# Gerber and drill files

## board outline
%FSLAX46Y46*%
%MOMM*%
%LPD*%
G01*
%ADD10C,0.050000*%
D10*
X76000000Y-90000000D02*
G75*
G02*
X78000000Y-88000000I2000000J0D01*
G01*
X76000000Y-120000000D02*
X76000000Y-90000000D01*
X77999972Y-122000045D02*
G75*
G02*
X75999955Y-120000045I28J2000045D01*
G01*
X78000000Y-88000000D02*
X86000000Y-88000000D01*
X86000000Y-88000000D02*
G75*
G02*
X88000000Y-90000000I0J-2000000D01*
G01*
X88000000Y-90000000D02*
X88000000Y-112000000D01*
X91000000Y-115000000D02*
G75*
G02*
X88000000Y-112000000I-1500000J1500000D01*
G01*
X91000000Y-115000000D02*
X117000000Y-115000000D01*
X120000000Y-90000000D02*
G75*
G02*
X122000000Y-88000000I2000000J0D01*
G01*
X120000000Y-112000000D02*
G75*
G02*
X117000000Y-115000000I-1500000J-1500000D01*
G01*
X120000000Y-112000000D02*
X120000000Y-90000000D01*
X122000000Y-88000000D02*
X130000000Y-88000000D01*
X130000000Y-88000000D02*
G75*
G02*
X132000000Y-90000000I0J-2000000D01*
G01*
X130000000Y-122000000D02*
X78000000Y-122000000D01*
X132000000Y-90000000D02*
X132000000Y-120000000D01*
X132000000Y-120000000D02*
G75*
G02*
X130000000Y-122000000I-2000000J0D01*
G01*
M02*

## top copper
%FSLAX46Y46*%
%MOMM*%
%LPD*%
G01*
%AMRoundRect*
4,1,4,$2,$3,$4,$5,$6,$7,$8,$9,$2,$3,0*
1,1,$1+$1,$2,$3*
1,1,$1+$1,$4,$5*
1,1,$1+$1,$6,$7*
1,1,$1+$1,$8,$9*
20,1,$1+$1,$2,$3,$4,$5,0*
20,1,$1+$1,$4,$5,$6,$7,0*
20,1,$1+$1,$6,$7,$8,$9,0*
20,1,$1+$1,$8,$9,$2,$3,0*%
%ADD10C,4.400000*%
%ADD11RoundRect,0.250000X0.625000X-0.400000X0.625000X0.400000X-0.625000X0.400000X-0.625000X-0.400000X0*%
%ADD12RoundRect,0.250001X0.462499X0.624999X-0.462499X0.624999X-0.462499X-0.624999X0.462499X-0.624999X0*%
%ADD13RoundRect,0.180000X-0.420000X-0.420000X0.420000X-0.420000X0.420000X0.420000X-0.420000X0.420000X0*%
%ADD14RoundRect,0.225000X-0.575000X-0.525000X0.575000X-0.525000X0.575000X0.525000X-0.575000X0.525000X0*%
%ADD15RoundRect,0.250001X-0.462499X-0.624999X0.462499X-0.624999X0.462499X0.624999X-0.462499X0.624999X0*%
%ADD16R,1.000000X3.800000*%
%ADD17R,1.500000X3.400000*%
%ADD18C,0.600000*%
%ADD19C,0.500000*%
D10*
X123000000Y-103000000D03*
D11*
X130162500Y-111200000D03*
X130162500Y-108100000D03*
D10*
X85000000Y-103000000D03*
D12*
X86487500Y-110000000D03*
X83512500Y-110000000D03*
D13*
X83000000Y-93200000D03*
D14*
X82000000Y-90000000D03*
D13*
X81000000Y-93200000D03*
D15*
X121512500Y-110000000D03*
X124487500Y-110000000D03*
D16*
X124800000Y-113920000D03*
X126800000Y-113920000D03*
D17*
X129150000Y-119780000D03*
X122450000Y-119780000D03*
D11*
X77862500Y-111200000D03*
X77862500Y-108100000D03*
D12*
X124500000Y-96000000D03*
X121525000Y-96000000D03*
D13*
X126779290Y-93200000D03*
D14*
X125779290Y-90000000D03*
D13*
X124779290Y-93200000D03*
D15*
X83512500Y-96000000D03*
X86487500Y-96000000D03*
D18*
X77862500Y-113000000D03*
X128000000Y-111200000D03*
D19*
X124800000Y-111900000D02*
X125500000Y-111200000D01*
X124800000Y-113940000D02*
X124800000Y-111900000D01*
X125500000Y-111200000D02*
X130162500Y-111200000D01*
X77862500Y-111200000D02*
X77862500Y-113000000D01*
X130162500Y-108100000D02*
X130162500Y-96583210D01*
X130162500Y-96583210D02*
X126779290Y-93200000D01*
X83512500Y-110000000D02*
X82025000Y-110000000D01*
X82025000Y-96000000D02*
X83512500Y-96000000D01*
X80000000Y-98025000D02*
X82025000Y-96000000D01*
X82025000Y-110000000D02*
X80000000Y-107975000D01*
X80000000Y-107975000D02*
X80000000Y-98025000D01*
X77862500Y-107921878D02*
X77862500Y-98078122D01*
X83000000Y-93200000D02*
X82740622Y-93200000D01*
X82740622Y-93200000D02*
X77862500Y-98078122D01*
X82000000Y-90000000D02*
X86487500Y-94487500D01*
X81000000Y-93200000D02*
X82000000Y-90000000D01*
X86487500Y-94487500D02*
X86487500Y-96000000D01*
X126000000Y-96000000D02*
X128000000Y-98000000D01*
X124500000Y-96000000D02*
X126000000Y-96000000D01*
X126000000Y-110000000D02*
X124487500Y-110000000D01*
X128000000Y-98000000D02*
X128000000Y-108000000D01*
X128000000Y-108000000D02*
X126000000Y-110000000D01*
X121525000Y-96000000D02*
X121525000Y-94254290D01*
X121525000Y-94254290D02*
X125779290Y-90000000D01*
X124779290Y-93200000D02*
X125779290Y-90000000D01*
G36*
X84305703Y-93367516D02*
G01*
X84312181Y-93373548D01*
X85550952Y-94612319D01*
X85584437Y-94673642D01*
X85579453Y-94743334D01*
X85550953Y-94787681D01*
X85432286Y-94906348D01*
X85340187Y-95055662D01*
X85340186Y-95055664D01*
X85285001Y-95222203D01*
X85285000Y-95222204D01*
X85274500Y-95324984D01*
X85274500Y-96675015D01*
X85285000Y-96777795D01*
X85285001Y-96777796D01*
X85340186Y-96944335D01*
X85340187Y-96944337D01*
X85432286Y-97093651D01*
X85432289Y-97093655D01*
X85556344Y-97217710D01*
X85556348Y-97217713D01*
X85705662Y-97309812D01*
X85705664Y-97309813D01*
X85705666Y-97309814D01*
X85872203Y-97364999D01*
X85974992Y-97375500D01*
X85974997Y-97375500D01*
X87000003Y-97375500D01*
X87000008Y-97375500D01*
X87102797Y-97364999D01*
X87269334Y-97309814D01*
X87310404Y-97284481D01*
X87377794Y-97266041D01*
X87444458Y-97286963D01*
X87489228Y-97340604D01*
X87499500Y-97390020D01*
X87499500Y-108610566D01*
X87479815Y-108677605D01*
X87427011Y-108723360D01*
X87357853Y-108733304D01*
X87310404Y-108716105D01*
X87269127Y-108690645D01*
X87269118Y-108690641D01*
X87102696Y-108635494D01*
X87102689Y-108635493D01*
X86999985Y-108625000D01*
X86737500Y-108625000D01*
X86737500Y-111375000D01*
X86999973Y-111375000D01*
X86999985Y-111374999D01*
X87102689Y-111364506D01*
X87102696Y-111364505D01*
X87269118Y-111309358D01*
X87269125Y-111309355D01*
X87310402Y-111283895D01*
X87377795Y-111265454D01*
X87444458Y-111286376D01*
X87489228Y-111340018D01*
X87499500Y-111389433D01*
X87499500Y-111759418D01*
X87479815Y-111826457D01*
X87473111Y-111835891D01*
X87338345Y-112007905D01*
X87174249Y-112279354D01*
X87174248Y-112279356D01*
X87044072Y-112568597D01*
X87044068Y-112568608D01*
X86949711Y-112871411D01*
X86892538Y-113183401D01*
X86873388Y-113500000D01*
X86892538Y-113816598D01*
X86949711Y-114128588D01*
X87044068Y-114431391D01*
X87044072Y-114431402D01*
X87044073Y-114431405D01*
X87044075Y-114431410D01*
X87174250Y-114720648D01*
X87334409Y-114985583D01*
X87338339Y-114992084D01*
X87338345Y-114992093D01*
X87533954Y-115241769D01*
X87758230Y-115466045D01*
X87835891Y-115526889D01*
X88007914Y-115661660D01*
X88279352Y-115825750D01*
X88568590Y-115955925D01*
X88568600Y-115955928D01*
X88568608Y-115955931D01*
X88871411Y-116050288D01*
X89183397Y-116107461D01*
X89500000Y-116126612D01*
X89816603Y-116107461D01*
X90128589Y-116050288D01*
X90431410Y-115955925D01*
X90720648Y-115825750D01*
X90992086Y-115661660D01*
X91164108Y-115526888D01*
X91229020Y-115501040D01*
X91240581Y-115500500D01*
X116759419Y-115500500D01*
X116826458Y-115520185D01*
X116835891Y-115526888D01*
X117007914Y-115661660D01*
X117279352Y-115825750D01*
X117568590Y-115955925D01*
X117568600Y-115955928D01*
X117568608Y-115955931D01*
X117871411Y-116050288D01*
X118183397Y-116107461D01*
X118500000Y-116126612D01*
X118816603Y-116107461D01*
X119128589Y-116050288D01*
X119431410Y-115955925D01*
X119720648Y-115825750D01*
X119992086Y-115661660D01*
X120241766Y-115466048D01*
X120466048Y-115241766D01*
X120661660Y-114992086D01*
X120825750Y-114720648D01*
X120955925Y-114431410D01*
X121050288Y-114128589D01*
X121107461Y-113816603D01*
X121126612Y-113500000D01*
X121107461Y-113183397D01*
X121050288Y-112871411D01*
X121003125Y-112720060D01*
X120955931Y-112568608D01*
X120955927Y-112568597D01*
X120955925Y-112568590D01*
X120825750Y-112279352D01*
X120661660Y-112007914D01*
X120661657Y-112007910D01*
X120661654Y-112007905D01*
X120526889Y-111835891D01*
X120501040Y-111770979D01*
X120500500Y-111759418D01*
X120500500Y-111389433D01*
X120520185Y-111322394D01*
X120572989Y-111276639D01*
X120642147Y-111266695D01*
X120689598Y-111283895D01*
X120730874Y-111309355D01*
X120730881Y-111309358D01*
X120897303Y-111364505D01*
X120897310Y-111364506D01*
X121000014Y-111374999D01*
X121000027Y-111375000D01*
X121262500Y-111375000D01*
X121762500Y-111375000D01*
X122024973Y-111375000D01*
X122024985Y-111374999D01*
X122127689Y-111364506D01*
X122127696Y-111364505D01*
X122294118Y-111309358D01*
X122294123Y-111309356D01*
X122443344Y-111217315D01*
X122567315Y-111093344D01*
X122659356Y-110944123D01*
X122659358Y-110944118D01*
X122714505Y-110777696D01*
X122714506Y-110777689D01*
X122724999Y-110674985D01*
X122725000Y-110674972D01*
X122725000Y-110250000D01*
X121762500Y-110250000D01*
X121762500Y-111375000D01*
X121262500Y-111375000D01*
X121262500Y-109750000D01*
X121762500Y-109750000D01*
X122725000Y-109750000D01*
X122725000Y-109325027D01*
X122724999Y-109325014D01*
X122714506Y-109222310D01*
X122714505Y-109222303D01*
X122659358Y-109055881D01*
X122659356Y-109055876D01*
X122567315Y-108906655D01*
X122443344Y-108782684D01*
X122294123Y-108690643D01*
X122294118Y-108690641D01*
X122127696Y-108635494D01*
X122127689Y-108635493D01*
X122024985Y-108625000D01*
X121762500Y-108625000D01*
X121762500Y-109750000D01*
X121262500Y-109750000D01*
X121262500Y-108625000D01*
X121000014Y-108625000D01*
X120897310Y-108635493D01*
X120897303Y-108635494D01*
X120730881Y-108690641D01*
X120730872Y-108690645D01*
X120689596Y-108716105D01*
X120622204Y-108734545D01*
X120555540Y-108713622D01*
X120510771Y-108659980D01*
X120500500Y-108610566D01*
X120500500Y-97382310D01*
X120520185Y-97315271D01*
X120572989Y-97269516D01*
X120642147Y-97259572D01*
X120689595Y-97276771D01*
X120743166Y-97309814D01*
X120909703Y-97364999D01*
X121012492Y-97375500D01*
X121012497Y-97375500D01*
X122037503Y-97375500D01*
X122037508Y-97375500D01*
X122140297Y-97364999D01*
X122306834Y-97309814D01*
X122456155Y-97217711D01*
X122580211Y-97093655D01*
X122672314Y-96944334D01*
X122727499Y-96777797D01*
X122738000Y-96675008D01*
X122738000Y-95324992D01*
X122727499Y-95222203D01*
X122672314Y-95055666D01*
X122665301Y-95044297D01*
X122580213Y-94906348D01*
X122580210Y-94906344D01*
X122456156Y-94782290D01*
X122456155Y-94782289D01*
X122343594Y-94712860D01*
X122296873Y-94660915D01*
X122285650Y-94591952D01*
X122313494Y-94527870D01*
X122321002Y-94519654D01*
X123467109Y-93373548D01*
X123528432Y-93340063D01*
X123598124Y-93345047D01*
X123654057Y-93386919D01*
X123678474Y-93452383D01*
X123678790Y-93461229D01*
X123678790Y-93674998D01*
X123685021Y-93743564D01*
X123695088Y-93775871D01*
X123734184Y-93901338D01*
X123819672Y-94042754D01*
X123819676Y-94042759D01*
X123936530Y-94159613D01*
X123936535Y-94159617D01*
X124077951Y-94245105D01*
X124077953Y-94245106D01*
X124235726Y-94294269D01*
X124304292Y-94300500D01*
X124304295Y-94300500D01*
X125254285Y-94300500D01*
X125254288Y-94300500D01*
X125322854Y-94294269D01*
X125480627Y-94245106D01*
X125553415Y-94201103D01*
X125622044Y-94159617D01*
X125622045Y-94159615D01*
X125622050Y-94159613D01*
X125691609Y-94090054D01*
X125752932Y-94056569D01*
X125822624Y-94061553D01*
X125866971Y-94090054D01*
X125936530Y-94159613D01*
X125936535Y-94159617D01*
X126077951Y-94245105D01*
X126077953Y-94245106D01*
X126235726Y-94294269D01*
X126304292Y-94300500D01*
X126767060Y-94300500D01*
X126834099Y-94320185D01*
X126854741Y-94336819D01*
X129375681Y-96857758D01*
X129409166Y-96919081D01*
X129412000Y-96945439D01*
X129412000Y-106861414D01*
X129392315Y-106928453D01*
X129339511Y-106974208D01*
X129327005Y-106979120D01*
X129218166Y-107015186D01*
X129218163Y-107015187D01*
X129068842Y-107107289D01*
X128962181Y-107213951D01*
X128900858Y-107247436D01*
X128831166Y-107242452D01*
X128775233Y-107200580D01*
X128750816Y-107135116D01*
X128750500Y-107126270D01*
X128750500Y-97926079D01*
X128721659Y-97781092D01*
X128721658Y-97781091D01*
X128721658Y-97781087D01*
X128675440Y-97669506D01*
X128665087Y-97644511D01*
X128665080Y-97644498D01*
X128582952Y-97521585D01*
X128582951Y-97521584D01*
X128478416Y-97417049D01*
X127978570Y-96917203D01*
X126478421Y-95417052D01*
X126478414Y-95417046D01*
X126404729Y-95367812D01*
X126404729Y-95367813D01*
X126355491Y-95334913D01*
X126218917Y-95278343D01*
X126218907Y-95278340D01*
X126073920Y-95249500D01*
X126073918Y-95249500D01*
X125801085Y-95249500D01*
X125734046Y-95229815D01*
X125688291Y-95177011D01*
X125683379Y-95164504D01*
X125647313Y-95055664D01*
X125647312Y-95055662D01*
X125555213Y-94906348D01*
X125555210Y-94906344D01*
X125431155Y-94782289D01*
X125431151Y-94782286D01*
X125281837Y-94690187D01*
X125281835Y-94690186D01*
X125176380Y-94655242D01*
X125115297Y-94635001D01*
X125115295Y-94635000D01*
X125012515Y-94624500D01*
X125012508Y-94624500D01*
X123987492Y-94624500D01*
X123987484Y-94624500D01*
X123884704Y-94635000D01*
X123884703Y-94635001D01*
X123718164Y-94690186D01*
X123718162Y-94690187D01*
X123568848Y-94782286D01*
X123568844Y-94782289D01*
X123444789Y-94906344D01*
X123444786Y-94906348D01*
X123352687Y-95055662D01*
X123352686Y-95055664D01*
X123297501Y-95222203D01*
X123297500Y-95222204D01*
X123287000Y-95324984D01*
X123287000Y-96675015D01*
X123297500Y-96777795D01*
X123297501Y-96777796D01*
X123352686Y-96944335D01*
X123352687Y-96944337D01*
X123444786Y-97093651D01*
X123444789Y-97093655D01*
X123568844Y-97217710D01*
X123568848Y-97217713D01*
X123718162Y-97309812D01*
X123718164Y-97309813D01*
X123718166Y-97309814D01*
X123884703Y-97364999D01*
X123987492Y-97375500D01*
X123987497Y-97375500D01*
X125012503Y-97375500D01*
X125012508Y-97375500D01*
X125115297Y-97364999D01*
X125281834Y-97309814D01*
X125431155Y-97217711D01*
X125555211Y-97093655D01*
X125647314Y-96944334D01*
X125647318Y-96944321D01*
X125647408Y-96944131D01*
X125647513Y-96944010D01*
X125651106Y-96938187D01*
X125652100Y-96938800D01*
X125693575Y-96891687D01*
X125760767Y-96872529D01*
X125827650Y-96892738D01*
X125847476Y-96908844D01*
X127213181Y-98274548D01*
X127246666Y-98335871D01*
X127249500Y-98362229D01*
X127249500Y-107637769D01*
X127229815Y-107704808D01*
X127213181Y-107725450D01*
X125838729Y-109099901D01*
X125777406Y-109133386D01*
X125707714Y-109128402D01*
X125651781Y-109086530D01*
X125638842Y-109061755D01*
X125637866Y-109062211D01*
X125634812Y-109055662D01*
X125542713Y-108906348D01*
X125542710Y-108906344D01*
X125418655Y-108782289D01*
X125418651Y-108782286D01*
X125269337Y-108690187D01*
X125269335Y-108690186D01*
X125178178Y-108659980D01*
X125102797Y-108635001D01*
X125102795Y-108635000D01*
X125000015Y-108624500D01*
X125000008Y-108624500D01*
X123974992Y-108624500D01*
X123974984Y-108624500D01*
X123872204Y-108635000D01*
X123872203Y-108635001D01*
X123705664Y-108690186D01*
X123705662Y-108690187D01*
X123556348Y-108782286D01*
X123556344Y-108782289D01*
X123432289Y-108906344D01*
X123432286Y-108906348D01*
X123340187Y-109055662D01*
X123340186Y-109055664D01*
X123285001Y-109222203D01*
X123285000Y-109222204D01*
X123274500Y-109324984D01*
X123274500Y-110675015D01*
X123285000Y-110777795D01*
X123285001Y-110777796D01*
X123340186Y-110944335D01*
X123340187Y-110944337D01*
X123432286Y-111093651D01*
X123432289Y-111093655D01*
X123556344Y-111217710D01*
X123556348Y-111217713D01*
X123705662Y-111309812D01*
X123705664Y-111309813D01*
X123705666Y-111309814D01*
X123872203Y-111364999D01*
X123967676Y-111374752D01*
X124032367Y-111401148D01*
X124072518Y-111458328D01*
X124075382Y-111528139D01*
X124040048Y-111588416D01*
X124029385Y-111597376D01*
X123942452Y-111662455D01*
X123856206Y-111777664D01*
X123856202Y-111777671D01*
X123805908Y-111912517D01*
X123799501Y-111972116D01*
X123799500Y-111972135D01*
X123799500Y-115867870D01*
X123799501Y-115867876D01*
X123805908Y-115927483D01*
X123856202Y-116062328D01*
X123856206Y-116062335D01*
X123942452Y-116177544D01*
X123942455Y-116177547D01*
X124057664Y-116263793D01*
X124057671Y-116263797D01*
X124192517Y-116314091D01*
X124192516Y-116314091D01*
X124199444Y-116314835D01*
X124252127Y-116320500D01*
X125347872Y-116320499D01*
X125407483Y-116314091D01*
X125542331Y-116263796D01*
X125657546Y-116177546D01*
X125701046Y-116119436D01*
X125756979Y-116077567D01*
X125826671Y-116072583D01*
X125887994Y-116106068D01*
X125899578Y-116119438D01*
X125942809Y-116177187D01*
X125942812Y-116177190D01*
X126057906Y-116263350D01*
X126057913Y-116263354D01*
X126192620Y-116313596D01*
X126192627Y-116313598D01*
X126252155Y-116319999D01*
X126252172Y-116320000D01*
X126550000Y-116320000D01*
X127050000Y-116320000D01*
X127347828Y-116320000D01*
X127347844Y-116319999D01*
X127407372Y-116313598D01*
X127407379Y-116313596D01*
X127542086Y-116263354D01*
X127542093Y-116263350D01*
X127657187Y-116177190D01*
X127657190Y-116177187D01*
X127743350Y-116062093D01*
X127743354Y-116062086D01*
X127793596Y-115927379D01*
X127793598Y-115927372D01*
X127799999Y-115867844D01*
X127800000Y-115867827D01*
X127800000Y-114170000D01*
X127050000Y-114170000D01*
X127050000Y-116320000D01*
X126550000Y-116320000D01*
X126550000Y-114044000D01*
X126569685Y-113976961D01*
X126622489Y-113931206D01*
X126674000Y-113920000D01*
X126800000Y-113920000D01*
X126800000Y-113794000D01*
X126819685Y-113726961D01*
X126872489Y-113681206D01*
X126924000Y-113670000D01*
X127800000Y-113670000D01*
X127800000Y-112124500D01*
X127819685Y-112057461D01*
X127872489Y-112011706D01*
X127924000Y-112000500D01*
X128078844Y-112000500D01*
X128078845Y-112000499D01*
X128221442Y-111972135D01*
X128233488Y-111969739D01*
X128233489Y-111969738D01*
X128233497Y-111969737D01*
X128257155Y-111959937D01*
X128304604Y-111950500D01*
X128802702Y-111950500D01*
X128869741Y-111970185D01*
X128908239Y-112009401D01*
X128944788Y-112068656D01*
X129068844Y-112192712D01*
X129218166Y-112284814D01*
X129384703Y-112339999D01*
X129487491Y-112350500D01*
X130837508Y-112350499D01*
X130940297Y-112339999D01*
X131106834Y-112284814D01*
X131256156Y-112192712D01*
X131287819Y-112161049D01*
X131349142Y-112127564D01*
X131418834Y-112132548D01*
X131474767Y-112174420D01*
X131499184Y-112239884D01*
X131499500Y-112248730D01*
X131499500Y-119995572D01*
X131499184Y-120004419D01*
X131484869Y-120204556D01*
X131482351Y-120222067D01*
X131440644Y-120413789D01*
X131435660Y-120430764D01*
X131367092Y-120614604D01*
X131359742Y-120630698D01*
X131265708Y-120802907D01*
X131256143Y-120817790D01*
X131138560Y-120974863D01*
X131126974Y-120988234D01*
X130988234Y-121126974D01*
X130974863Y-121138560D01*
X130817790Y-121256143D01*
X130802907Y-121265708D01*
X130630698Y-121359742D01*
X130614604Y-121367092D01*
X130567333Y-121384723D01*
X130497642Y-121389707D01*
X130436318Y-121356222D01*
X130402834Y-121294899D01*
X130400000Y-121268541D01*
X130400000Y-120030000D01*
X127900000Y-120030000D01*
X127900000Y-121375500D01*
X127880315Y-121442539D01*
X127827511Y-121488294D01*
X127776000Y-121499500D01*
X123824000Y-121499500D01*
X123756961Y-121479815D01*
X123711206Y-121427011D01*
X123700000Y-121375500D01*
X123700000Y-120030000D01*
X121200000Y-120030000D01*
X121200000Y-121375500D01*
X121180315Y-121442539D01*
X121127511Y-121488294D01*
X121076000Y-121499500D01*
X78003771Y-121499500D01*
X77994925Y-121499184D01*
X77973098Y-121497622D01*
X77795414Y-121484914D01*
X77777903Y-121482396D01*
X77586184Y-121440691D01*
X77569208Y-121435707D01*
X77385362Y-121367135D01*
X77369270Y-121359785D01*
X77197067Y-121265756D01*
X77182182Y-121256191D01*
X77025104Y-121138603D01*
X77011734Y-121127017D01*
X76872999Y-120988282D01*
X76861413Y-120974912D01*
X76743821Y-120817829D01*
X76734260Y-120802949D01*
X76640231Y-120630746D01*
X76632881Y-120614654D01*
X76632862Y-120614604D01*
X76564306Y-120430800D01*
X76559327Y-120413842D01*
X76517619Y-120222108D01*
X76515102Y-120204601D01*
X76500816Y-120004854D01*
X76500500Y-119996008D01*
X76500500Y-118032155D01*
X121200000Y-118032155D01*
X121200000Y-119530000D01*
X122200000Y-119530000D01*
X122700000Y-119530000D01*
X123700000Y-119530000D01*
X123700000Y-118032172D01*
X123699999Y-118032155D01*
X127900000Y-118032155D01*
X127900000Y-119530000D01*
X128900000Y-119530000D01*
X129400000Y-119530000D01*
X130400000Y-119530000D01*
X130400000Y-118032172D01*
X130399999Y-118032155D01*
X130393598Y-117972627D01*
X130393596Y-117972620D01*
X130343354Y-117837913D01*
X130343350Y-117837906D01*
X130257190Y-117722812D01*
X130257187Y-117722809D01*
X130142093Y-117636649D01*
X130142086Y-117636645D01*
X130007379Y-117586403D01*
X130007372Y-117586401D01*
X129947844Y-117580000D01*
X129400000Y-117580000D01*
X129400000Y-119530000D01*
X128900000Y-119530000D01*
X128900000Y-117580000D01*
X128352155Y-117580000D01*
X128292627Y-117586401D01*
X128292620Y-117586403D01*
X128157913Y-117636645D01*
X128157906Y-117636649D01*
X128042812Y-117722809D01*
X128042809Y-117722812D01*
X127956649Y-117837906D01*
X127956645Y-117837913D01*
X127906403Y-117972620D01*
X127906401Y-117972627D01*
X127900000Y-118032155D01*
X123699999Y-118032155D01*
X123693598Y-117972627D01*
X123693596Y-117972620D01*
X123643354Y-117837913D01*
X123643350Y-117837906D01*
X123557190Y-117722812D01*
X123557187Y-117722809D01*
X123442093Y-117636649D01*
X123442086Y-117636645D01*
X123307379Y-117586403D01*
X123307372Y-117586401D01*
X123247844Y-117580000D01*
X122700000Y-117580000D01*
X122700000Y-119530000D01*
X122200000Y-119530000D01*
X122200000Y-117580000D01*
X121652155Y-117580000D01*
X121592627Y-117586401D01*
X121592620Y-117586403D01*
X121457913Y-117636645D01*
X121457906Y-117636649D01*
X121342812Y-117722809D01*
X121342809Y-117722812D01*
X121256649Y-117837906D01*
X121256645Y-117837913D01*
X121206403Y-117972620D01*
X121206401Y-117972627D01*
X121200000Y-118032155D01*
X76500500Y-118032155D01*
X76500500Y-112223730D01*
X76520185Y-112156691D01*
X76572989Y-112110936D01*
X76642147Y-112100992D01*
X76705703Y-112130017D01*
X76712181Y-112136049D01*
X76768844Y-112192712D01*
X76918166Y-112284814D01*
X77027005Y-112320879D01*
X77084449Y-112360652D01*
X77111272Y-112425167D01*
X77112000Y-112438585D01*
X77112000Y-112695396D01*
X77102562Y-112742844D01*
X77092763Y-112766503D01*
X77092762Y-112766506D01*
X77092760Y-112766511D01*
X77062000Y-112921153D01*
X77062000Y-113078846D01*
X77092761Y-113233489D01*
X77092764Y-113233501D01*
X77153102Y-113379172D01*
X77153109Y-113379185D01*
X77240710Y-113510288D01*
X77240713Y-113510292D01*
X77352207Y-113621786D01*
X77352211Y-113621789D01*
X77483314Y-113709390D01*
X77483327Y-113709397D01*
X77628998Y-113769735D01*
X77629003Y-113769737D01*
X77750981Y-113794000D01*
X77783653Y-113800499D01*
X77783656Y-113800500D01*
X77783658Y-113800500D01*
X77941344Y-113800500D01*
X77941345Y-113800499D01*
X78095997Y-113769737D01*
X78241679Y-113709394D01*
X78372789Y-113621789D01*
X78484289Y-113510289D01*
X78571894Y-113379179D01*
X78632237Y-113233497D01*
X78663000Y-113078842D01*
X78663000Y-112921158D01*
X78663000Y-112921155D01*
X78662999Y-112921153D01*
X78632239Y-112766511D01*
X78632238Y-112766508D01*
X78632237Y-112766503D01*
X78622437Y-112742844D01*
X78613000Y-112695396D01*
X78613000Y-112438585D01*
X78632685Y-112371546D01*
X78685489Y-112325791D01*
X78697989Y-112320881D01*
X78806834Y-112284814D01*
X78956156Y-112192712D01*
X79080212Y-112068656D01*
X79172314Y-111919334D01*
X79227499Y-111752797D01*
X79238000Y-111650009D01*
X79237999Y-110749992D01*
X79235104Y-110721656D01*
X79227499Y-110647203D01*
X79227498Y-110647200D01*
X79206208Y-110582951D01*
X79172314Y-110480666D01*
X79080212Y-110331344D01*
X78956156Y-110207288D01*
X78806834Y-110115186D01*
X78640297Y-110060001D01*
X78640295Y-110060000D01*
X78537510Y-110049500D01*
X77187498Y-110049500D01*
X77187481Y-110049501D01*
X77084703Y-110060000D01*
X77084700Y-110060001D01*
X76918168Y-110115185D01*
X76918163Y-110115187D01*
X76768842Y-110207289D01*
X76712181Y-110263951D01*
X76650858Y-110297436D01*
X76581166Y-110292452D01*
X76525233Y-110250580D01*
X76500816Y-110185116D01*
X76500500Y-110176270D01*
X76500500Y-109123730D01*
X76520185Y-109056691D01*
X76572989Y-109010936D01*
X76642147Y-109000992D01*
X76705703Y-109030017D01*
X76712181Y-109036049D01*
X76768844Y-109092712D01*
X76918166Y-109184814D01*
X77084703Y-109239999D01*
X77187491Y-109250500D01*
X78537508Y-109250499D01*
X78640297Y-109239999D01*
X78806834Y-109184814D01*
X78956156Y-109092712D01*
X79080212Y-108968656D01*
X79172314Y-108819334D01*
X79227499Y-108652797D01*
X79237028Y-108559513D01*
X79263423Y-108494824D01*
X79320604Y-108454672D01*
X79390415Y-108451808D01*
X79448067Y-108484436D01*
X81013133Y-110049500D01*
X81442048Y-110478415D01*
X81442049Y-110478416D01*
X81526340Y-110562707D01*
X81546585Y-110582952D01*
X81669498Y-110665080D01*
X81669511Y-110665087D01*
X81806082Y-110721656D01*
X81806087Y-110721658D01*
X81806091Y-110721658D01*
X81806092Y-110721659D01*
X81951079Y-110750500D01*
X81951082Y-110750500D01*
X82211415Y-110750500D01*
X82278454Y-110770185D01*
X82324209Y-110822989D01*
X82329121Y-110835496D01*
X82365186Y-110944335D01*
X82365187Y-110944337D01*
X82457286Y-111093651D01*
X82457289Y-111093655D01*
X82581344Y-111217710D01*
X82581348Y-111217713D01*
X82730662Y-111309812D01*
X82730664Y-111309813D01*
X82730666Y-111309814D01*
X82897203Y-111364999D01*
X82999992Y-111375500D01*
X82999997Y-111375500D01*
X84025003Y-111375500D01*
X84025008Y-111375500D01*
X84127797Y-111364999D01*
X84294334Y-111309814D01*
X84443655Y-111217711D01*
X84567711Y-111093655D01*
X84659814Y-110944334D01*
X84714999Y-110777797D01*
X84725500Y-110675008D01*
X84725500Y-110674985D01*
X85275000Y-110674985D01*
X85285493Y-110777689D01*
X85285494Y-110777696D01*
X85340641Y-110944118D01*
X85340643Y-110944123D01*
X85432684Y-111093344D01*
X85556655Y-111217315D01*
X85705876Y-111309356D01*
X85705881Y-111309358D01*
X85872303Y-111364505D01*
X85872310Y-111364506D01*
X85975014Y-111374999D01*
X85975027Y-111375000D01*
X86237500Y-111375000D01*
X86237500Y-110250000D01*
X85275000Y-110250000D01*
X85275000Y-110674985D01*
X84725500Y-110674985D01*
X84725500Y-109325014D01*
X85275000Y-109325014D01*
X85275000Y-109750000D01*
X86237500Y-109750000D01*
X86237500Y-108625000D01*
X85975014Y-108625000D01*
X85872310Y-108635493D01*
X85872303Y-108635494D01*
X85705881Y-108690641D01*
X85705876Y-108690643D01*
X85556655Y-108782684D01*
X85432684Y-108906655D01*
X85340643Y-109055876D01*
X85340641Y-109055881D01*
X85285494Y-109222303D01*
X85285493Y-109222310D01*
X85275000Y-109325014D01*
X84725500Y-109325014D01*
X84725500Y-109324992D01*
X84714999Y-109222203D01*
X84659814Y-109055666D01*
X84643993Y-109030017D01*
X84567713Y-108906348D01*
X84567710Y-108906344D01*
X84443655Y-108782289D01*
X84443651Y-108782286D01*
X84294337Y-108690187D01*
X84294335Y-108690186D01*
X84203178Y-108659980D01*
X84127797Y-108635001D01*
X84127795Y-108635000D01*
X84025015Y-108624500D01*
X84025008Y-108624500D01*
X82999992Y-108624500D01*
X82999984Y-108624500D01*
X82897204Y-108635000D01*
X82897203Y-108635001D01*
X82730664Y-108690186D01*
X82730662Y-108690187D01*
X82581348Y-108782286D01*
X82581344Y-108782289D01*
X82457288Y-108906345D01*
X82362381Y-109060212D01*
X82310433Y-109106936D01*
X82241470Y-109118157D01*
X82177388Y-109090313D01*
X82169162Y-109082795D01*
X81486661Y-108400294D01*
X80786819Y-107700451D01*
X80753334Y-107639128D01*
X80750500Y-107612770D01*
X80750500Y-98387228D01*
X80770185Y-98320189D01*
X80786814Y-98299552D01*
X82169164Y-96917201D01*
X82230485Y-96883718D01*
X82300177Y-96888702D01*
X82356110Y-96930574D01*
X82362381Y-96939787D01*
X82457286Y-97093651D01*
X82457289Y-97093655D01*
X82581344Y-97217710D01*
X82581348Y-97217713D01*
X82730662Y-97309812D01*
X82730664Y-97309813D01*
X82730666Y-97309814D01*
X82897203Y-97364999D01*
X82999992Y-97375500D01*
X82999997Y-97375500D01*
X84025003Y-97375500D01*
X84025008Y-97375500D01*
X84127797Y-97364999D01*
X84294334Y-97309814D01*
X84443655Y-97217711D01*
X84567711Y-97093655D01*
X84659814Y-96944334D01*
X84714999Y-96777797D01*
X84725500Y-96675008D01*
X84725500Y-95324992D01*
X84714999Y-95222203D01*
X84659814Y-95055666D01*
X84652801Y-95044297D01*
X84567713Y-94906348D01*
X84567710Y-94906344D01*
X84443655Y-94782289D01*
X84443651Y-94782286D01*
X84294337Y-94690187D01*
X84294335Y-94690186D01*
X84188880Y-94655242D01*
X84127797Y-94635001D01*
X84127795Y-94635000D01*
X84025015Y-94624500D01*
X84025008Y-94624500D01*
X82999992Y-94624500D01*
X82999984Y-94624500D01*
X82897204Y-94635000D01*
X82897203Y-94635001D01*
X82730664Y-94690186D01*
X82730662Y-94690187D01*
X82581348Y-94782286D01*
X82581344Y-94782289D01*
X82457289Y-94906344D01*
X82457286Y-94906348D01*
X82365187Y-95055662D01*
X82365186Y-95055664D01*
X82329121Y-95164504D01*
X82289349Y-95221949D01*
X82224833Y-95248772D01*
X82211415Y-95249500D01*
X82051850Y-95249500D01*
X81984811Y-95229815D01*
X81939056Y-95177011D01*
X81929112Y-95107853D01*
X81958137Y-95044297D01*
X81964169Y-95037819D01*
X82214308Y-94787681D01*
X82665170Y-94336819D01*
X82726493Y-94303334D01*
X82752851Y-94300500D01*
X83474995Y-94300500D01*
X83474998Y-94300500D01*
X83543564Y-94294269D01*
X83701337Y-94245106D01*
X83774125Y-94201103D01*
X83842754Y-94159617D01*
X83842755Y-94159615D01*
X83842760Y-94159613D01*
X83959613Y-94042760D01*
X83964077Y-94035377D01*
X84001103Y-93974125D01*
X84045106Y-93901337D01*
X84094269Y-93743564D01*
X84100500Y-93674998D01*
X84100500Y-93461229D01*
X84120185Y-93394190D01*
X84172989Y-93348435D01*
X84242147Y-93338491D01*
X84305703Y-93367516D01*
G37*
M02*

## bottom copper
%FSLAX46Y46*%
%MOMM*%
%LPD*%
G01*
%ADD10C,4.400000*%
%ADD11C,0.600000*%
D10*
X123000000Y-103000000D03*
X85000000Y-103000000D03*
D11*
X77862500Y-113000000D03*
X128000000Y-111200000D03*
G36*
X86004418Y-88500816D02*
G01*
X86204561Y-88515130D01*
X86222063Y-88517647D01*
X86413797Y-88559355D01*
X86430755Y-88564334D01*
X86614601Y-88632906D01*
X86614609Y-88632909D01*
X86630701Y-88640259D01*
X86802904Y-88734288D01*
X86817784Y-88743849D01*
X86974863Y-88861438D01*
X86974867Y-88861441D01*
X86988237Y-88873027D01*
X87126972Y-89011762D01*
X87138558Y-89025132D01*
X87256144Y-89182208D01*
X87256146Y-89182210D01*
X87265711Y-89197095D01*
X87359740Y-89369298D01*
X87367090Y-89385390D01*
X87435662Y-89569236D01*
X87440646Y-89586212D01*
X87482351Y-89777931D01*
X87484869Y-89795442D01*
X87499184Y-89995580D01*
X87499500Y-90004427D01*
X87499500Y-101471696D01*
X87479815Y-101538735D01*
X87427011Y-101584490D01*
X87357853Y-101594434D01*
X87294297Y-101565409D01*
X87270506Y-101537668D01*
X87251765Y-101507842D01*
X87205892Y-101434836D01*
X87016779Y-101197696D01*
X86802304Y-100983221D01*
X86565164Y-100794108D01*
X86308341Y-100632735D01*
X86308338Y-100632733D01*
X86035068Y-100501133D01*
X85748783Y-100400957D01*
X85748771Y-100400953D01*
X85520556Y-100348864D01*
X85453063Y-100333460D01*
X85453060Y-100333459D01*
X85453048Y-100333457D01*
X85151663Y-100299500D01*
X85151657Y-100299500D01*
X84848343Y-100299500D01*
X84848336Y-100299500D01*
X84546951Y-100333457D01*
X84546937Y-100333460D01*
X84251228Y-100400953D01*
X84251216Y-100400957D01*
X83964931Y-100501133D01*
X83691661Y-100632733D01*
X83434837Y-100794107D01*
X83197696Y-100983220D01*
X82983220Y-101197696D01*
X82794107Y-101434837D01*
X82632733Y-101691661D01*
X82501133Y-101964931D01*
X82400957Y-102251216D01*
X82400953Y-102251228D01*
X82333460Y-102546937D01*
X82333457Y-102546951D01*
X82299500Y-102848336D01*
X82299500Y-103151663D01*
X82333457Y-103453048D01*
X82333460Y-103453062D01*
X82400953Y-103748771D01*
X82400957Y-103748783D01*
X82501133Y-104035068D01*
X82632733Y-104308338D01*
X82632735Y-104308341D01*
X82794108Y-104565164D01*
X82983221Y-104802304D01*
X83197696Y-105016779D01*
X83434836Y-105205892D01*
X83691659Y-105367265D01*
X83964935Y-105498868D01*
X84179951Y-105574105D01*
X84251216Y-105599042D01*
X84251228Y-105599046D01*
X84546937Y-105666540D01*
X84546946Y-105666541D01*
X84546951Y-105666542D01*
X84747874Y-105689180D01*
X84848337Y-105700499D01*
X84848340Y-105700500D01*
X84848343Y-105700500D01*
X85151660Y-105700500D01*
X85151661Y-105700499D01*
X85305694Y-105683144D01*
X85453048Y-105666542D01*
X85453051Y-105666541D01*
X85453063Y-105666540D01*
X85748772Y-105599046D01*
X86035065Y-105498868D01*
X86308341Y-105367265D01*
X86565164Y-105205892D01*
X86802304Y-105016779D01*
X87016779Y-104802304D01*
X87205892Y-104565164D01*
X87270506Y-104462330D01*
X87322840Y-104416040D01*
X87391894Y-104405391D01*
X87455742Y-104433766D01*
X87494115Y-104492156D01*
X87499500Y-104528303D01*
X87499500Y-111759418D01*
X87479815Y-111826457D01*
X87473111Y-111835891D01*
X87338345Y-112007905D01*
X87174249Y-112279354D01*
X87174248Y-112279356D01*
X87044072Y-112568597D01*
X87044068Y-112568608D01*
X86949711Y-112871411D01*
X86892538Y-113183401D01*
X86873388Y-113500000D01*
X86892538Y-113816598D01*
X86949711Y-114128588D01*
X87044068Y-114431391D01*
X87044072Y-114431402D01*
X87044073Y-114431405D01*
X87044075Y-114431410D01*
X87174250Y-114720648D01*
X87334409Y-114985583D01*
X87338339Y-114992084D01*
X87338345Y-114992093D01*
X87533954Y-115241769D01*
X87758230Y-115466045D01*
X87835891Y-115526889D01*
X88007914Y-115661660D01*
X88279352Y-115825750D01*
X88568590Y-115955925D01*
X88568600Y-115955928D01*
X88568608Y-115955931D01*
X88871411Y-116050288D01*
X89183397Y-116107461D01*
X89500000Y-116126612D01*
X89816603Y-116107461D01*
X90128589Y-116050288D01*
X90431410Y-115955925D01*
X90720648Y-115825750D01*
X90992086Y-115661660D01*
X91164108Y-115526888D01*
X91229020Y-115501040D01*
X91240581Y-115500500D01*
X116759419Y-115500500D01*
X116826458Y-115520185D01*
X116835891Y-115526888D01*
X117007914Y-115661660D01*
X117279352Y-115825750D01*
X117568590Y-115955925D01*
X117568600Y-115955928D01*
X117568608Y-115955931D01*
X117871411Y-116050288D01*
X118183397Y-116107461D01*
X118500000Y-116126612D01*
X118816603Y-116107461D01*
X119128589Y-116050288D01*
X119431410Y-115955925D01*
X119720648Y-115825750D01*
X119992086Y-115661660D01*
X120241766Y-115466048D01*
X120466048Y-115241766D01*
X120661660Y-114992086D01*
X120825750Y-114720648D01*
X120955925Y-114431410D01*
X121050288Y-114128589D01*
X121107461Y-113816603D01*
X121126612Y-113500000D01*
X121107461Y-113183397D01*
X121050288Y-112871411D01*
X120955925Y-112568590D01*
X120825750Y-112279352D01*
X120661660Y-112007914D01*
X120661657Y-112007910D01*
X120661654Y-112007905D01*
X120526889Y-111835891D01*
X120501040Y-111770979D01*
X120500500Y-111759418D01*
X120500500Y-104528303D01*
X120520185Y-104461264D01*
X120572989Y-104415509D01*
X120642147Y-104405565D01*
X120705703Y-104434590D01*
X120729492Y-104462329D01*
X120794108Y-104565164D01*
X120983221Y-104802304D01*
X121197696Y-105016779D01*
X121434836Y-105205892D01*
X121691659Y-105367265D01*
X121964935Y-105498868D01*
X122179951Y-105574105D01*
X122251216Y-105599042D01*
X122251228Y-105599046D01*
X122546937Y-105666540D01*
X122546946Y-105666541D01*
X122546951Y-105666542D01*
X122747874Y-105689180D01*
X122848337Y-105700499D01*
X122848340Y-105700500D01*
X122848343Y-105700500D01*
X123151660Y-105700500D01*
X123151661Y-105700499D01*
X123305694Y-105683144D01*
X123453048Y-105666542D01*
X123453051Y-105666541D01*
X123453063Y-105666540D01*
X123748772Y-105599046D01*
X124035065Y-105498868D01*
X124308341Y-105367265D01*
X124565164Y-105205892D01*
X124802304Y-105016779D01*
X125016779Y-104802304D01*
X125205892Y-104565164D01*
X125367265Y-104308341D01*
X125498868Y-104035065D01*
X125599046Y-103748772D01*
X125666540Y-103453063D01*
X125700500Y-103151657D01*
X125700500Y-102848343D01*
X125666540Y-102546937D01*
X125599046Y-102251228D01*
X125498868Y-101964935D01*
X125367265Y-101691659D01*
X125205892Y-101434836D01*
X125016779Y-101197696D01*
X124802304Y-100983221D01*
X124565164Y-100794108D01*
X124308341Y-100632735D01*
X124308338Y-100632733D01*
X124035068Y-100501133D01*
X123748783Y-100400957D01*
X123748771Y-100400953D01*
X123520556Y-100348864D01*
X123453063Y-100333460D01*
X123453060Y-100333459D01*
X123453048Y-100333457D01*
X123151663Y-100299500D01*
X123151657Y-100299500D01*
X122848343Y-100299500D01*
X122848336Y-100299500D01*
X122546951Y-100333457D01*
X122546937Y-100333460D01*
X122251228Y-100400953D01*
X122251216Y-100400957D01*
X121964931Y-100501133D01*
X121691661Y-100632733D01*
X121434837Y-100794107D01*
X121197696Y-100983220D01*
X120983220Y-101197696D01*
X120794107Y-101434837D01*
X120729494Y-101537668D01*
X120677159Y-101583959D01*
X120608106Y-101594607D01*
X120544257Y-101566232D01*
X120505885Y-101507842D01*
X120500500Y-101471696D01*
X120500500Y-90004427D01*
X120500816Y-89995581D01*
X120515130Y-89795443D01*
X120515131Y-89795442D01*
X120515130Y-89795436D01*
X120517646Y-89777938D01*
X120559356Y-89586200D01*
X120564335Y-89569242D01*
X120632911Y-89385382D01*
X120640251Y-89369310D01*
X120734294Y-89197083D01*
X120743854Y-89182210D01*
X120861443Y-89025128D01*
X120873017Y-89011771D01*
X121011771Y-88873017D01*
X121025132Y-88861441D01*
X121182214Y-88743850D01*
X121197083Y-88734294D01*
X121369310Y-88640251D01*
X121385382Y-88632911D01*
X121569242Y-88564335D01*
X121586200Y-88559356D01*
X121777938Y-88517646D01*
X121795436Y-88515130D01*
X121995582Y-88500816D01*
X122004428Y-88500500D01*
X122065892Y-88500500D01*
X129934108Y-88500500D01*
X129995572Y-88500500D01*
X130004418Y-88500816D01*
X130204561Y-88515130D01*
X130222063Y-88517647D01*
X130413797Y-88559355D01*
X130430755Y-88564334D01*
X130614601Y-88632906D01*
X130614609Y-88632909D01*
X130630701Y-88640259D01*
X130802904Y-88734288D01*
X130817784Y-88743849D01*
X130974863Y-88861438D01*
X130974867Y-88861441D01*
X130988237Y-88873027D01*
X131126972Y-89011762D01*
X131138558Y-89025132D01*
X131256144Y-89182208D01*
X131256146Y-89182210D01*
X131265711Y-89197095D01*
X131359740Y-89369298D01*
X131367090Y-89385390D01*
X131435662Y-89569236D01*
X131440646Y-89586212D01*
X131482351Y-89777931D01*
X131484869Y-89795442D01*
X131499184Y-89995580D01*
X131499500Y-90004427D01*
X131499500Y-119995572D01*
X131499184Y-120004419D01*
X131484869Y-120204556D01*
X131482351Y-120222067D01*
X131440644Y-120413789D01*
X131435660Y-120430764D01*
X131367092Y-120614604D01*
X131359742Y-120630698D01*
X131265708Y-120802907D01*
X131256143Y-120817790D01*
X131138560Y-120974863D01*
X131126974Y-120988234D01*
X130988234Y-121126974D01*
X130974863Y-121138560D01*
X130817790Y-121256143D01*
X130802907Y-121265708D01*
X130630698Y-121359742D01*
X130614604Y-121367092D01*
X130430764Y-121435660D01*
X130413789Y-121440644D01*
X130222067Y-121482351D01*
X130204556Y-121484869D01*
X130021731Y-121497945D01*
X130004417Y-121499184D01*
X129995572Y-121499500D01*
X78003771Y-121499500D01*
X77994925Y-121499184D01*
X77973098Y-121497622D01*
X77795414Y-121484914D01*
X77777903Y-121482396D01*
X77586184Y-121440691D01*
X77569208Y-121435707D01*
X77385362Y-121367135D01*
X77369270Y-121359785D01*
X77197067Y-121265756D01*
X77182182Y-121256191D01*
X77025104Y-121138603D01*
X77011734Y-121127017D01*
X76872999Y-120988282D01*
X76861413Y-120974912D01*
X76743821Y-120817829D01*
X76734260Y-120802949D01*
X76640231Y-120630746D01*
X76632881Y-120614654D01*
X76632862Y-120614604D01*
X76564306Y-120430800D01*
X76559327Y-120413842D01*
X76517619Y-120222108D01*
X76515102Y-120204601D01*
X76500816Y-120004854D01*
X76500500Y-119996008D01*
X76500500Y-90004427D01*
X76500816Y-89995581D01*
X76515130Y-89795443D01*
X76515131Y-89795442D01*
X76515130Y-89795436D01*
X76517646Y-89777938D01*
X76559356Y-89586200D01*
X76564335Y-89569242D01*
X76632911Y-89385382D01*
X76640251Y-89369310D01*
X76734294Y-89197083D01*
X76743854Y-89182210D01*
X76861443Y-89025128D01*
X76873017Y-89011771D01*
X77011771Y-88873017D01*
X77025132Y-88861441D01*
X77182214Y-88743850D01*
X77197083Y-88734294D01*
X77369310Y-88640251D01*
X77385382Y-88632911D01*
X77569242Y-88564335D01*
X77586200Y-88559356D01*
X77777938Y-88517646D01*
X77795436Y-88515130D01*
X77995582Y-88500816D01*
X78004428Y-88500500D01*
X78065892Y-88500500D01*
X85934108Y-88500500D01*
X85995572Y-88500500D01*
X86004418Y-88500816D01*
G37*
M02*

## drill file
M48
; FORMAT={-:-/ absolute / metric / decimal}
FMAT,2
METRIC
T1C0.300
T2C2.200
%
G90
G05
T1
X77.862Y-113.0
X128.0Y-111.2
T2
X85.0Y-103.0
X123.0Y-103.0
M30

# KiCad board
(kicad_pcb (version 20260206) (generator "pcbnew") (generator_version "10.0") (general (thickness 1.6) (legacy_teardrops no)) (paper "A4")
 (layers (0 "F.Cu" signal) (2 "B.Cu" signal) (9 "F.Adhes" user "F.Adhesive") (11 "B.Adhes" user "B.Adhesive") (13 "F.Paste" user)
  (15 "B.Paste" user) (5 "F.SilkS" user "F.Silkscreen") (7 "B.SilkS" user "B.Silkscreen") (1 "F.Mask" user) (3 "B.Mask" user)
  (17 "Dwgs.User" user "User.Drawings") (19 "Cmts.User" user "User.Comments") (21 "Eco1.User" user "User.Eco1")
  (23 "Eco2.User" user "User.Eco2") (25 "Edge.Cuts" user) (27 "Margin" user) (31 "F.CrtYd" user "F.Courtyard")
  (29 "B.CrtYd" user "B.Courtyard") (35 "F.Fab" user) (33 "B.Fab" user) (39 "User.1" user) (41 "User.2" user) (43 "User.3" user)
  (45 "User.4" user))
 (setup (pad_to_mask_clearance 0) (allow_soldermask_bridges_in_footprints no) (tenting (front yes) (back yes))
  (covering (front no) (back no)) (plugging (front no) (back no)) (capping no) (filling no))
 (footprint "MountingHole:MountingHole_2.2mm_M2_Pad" (layer "F.Cu") (at 123 103)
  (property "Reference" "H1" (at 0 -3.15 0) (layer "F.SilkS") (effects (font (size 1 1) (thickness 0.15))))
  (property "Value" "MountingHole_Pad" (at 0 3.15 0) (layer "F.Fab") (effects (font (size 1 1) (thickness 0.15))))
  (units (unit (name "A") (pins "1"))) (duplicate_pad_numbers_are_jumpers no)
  (pad "1" thru_hole circle (at 0 0) (size 4.4 4.4) (drill 2.2) (layers "*.Cu" "*.Mask") (remove_unused_layers no) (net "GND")
   (zone_connect 2)))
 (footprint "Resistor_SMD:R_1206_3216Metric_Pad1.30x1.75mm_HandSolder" (layer "F.Cu") (at 130.1625 109.65 90)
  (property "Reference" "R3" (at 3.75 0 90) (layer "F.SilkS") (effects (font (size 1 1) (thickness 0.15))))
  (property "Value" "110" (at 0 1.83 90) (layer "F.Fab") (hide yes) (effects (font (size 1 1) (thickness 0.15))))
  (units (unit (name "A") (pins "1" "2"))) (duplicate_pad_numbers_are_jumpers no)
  (pad "1" smd roundrect (at -1.55 0 90) (size 1.3 1.75) (layers "F.Cu" "F.Mask" "F.Paste") (roundrect_rratio 0.192308) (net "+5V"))
  (pad "2" smd roundrect (at 1.55 0 90) (size 1.3 1.75) (layers "F.Cu" "F.Mask" "F.Paste") (roundrect_rratio 0.192308) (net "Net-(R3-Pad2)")))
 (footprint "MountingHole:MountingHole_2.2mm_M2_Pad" (layer "F.Cu") (at 85 103)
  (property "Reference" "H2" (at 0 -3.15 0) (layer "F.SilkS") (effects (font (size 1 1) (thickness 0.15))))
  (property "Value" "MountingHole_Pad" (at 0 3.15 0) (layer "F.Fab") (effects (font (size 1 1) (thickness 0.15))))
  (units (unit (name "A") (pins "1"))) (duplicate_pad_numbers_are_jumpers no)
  (pad "1" thru_hole circle (at 0 0) (size 4.4 4.4) (drill 2.2) (layers "*.Cu" "*.Mask") (remove_unused_layers no) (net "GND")
   (zone_connect 2)))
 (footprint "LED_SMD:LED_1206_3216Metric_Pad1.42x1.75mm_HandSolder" (layer "F.Cu") (at 85 110 180)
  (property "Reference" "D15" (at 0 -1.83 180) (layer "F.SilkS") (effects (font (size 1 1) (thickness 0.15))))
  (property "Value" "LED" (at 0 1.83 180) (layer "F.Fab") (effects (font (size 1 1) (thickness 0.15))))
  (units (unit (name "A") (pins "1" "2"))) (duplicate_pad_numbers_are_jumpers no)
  (pad "1" smd roundrect (at -1.4875 0 180) (size 1.425 1.75) (layers "F.Cu" "F.Mask" "F.Paste") (roundrect_rratio 0.175439) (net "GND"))
  (pad "2" smd roundrect (at 1.4875 0 180) (size 1.425 1.75) (layers "F.Cu" "F.Mask" "F.Paste") (roundrect_rratio 0.175439)
   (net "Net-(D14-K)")))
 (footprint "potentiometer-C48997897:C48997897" (layer "F.Cu") (at 82 95.4)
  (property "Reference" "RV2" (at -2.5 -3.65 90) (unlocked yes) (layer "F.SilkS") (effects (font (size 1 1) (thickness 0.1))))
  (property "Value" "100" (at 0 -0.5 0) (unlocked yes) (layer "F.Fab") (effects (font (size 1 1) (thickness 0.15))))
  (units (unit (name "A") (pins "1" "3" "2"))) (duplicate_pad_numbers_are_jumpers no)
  (pad "1" smd roundrect (at 1 -2.2) (size 1.2 1.2) (layers "F.Cu" "F.Mask" "F.Paste") (roundrect_rratio 0.15) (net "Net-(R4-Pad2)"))
  (pad "2" smd roundrect (at 0 -5.4) (size 1.6 1.5) (layers "F.Cu" "F.Mask" "F.Paste") (roundrect_rratio 0.15) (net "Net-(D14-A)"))
  (pad "3" smd roundrect (at -1 -2.2) (size 1.2 1.2) (layers "F.Cu" "F.Mask" "F.Paste") (roundrect_rratio 0.15) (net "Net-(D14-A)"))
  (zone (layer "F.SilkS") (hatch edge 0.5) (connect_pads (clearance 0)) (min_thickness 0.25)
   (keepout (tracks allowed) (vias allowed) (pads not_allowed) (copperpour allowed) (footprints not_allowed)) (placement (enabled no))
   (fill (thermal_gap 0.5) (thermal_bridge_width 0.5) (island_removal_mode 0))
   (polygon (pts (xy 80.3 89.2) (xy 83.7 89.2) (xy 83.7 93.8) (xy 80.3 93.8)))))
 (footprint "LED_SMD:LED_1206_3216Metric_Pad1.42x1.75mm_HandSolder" (layer "F.Cu") (at 123 110)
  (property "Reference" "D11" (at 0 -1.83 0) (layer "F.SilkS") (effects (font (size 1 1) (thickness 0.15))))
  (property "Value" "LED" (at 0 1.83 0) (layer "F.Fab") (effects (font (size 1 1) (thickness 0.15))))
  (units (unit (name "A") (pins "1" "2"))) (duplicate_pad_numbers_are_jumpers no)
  (pad "1" smd roundrect (at -1.4875 0) (size 1.425 1.75) (layers "F.Cu" "F.Mask" "F.Paste") (roundrect_rratio 0.175439) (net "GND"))
  (pad "2" smd roundrect (at 1.4875 0) (size 1.425 1.75) (layers "F.Cu" "F.Mask" "F.Paste") (roundrect_rratio 0.175439) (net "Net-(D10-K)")))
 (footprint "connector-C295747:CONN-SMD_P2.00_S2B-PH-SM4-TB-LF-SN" (layer "F.Cu") (at 125.8 116.85)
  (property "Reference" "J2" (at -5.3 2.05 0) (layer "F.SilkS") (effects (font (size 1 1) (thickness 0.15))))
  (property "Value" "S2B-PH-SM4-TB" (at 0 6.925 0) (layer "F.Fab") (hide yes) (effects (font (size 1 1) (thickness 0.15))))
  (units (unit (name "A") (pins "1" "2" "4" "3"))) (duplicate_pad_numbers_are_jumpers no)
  (pad "1" smd rect (at -1 -2.93) (size 1 3.8) (layers "F.Cu" "F.Mask" "F.Paste") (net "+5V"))
  (pad "2" smd rect (at 1 -2.93) (size 1 3.8) (layers "F.Cu" "F.Mask" "F.Paste") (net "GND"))
  (pad "3" smd rect (at 3.35 2.93) (size 1.5 3.4) (layers "F.Cu" "F.Mask" "F.Paste") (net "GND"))
  (pad "4" smd rect (at -3.35 2.93) (size 1.5 3.4) (layers "F.Cu" "F.Mask" "F.Paste") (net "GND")))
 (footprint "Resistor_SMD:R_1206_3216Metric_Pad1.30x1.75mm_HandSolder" (layer "F.Cu") (at 77.8625 109.65 90)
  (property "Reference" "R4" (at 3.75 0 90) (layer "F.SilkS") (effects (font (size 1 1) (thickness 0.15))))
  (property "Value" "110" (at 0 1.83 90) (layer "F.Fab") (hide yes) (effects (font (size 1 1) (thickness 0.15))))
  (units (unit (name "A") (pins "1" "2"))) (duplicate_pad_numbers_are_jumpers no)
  (pad "1" smd roundrect (at -1.55 0 90) (size 1.3 1.75) (layers "F.Cu" "F.Mask" "F.Paste") (roundrect_rratio 0.192308) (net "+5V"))
  (pad "2" smd roundrect (at 1.55 0 90) (size 1.3 1.75) (layers "F.Cu" "F.Mask" "F.Paste") (roundrect_rratio 0.192308) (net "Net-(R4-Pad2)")))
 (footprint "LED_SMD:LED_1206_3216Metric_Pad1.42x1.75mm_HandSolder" (layer "F.Cu") (at 123.0125 96 180)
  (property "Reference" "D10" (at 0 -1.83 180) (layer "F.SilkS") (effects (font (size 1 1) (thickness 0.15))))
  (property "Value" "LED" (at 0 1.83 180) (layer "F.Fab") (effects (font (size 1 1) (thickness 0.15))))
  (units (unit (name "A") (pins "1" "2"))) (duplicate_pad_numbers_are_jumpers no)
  (pad "1" smd roundrect (at -1.4875 0 180) (size 1.425 1.75) (layers "F.Cu" "F.Mask" "F.Paste") (roundrect_rratio 0.175439)
   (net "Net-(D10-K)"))
  (pad "2" smd roundrect (at 1.4875 0 180) (size 1.425 1.75) (layers "F.Cu" "F.Mask" "F.Paste") (roundrect_rratio 0.175439)
   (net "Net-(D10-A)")))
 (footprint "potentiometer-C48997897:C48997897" (layer "F.Cu") (at 125.77929 95.4)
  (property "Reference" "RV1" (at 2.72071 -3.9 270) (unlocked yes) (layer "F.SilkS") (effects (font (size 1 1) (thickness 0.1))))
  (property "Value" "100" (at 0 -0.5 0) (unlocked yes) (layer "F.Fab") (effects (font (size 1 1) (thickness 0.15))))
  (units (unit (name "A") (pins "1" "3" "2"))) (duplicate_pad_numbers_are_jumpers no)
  (pad "1" smd roundrect (at 1 -2.2) (size 1.2 1.2) (layers "F.Cu" "F.Mask" "F.Paste") (roundrect_rratio 0.15) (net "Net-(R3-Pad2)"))
  (pad "2" smd roundrect (at 0 -5.4) (size 1.6 1.5) (layers "F.Cu" "F.Mask" "F.Paste") (roundrect_rratio 0.15) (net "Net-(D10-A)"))
  (pad "3" smd roundrect (at -1 -2.2) (size 1.2 1.2) (layers "F.Cu" "F.Mask" "F.Paste") (roundrect_rratio 0.15) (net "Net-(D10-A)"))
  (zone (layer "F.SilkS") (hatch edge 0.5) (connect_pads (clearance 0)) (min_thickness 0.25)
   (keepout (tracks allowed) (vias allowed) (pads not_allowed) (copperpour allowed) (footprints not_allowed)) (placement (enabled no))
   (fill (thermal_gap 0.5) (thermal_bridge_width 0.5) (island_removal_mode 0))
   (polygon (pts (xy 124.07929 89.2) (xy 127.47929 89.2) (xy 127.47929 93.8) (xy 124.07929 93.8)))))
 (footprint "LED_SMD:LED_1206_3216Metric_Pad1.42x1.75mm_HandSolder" (layer "F.Cu") (at 85 96)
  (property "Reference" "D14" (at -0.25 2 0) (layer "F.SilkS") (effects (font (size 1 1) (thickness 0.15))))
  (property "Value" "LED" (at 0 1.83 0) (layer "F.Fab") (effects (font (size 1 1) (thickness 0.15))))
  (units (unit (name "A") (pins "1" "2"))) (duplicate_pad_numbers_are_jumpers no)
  (pad "1" smd roundrect (at -1.4875 0) (size 1.425 1.75) (layers "F.Cu" "F.Mask" "F.Paste") (roundrect_rratio 0.175439) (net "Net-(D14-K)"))
  (pad "2" smd roundrect (at 1.4875 0) (size 1.425 1.75) (layers "F.Cu" "F.Mask" "F.Paste") (roundrect_rratio 0.175439) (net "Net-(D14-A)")))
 (gr_arc (start 76 90) (mid 76.585786 88.585786) (end 78 88) (stroke (width 0.05) (type default)) (layer "Edge.Cuts"))
 (gr_line (start 76 120) (end 76 90) (stroke (width 0.05) (type default)) (layer "Edge.Cuts"))
 (gr_arc (start 77.999972 122.000045) (mid 76.585758 121.414258) (end 75.999972 120.000045) (stroke (width 0.05) (type default))
  (layer "Edge.Cuts"))
 (gr_line (start 78 88) (end 86 88) (stroke (width 0.05) (type default)) (layer "Edge.Cuts"))
 (gr_arc (start 86 88) (mid 87.414213 88.585786) (end 88 90) (stroke (width 0.05) (type default)) (layer "Edge.Cuts"))
 (gr_line (start 88 90) (end 88 112) (stroke (width 0.05) (type default)) (layer "Edge.Cuts"))
 (gr_arc (start 91 115) (mid 88 115) (end 88 112) (stroke (width 0.05) (type default)) (layer "Edge.Cuts"))
 (gr_line (start 91 115) (end 117 115) (stroke (width 0.05) (type default)) (layer "Edge.Cuts"))
 (gr_arc (start 120 90) (mid 120.585786 88.585786) (end 122 88) (stroke (width 0.05) (type default)) (layer "Edge.Cuts"))
 (gr_arc (start 120 112) (mid 120 115) (end 117 115) (stroke (width 0.05) (type default)) (layer "Edge.Cuts"))
 (gr_line (start 120 112) (end 120 90) (stroke (width 0.05) (type default)) (layer "Edge.Cuts"))
 (gr_line (start 122 88) (end 130 88) (stroke (width 0.05) (type default)) (layer "Edge.Cuts"))
 (gr_arc (start 130 88) (mid 131.414213 88.585786) (end 132 90) (stroke (width 0.05) (type default)) (layer "Edge.Cuts"))
 (gr_line (start 130 122) (end 78 122) (stroke (width 0.05) (type default)) (layer "Edge.Cuts"))
 (gr_line (start 132 90) (end 132 120) (stroke (width 0.05) (type default)) (layer "Edge.Cuts"))
 (gr_arc (start 132 120) (mid 131.414213 121.414213) (end 130 122) (stroke (width 0.05) (type default)) (layer "Edge.Cuts"))
 (segment (start 124.8 111.9) (end 125.5 111.2) (width 0.5) (layer "F.Cu") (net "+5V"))
 (segment (start 124.8 113.94) (end 124.8 111.9) (width 0.5) (layer "F.Cu") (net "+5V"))
 (segment (start 125.5 111.2) (end 130.1625 111.2) (width 0.5) (layer "F.Cu") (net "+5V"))
 (segment (start 77.8625 111.2) (end 77.8625 113) (width 0.5) (layer "F.Cu") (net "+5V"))
 (via (at 77.8625 113) (size 0.6) (drill 0.3) (layers "F.Cu" "B.Cu") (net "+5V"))
 (via (at 128 111.2) (size 0.6) (drill 0.3) (layers "F.Cu" "B.Cu") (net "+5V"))
 (segment (start 130.1625 108.1) (end 130.1625 96.58321) (width 0.5) (layer "F.Cu") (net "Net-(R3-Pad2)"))
 (segment (start 130.1625 96.58321) (end 126.77929 93.2) (width 0.5) (layer "F.Cu") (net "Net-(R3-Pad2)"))
 (segment (start 83.5125 110) (end 82.025 110) (width 0.5) (layer "F.Cu") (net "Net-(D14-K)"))
 (segment (start 82.025 96) (end 83.5125 96) (width 0.5) (layer "F.Cu") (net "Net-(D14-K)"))
 (segment (start 80 98.025) (end 82.025 96) (width 0.5) (layer "F.Cu") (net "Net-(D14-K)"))
 (segment (start 82.025 110) (end 80 107.975) (width 0.5) (layer "F.Cu") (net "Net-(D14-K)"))
 (segment (start 80 107.975) (end 80 98.025) (width 0.5) (layer "F.Cu") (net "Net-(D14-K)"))
 (segment (start 77.8625 107.921878) (end 77.8625 98.078122) (width 0.5) (layer "F.Cu") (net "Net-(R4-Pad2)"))
 (segment (start 83 93.2) (end 82.740622 93.2) (width 0.5) (layer "F.Cu") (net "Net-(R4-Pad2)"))
 (segment (start 82.740622 93.2) (end 77.8625 98.078122) (width 0.5) (layer "F.Cu") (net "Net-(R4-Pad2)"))
 (segment (start 82 90) (end 86.4875 94.4875) (width 0.5) (layer "F.Cu") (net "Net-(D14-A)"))
 (segment (start 81 93.2) (end 82 90) (width 0.5) (layer "F.Cu") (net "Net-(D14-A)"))
 (segment (start 86.4875 94.4875) (end 86.4875 96) (width 0.5) (layer "F.Cu") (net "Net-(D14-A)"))
 (segment (start 126 96) (end 128 98) (width 0.5) (layer "F.Cu") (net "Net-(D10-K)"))
 (segment (start 124.5 96) (end 126 96) (width 0.5) (layer "F.Cu") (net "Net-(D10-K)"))
 (segment (start 126 110) (end 124.4875 110) (width 0.5) (layer "F.Cu") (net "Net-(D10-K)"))
 (segment (start 128 98) (end 128 108) (width 0.5) (layer "F.Cu") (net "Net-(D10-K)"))
 (segment (start 128 108) (end 126 110) (width 0.5) (layer "F.Cu") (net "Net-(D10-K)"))
 (segment (start 121.525 96) (end 121.525 94.25429) (width 0.5) (layer "F.Cu") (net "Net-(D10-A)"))
 (segment (start 121.525 94.25429) (end 125.77929 90) (width 0.5) (layer "F.Cu") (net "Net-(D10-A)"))
 (segment (start 124.77929 93.2) (end 125.77929 90) (width 0.5) (layer "F.Cu") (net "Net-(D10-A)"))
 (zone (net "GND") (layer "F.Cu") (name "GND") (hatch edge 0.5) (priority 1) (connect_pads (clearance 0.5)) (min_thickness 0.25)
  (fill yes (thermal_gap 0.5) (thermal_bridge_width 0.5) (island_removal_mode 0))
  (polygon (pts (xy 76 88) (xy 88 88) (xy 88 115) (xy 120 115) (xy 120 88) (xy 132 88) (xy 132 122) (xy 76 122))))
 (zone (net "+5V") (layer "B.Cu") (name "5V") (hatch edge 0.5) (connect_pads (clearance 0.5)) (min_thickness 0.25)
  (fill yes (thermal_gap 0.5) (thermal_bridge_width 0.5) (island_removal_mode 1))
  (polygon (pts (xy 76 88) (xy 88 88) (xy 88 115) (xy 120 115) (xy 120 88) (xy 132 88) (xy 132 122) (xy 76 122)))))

